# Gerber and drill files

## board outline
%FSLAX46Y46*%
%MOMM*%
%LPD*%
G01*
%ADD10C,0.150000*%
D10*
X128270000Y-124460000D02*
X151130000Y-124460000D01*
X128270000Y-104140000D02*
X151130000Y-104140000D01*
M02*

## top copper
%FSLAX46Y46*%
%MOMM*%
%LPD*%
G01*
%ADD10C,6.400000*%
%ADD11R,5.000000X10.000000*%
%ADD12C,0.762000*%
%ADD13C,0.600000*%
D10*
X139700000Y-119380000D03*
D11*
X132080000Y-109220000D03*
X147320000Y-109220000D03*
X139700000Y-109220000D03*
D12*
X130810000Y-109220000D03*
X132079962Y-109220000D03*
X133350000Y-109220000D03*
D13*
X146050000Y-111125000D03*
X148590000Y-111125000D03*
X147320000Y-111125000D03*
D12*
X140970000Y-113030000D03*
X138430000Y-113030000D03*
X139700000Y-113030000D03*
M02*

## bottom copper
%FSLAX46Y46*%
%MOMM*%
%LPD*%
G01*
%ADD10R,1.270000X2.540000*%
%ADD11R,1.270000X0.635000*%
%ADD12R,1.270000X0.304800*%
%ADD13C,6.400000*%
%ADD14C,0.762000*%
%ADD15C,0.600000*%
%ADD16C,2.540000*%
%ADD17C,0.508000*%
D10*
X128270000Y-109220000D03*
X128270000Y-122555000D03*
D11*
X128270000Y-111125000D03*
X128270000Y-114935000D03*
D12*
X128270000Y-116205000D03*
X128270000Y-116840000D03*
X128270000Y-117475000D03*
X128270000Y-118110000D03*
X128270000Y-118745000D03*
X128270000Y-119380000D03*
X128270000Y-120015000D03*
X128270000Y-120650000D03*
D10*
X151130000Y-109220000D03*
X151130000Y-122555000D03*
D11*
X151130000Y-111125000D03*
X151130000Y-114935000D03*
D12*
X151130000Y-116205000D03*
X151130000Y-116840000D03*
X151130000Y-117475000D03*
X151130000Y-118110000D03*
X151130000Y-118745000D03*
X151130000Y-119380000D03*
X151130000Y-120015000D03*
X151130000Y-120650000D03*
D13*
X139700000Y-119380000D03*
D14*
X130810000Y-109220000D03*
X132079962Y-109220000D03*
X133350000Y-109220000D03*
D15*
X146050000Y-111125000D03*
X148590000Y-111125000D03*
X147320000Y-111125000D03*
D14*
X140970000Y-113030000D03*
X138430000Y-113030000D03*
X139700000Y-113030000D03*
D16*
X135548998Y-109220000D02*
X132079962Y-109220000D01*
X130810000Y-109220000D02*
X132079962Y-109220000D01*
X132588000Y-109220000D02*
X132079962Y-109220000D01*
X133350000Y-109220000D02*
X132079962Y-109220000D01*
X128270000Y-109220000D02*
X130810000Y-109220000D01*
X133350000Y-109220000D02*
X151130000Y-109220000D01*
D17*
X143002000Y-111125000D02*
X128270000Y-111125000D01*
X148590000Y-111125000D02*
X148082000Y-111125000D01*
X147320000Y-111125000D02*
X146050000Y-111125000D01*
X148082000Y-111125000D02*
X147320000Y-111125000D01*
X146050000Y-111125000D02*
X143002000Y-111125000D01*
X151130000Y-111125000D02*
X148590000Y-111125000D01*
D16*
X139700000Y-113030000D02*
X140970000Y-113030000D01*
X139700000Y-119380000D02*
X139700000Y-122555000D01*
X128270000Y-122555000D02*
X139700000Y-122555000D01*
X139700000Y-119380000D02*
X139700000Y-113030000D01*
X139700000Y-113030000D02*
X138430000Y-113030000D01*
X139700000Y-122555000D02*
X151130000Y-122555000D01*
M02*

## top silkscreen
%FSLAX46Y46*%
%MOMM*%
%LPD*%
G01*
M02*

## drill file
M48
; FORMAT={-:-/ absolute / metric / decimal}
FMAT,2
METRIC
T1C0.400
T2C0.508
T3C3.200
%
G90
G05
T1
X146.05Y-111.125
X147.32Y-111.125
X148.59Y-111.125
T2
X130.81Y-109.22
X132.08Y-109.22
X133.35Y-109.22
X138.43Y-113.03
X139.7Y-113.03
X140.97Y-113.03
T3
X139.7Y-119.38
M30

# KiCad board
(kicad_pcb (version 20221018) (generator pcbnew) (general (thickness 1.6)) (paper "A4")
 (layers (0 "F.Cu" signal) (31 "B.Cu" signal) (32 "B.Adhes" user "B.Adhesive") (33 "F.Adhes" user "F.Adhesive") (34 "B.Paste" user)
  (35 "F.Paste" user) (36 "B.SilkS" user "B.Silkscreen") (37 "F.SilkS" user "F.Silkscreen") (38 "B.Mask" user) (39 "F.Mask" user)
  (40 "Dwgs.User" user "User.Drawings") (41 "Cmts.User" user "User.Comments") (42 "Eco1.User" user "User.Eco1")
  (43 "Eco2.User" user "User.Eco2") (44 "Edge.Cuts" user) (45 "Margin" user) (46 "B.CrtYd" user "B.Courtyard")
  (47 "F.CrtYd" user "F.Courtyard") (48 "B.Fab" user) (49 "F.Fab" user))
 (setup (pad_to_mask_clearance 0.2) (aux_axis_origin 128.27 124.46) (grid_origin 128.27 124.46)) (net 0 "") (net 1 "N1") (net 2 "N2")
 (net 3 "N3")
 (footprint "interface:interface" (layer "F.Cu") (at 128.27 104.775)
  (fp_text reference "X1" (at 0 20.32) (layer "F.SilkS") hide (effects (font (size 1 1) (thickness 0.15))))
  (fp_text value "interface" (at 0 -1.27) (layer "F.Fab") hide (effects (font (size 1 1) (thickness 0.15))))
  (pad "1" smd rect (at 0 4.445) (size 1.27 2.54) (layers "B.Cu") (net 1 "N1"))
  (pad "2" smd rect (at 0 17.78) (size 1.27 2.54) (layers "B.Cu") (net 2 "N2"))
  (pad "3" smd rect (at 0 6.35) (size 1.27 0.635) (layers "B.Cu") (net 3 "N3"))
  (pad "4" smd rect (at 0 10.16) (size 1.27 0.635) (layers "B.Cu"))
  (pad "5" smd rect (at 0 11.43) (size 1.27 0.3048) (layers "B.Cu"))
  (pad "6" smd rect (at 0 12.065) (size 1.27 0.3048) (layers "B.Cu"))
  (pad "7" smd rect (at 0 12.7) (size 1.27 0.3048) (layers "B.Cu"))
  (pad "8" smd rect (at 0 13.335) (size 1.27 0.3048) (layers "B.Cu"))
  (pad "9" smd rect (at 0 13.97) (size 1.27 0.3048) (layers "B.Cu"))
  (pad "10" smd rect (at 0 14.605) (size 1.27 0.3048) (layers "B.Cu"))
  (pad "11" smd rect (at 0 15.24) (size 1.27 0.3048) (layers "B.Cu"))
  (pad "12" smd rect (at 0 15.875) (size 1.27 0.3048) (layers "B.Cu")))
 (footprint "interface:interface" (layer "F.Cu") (at 151.13 104.775)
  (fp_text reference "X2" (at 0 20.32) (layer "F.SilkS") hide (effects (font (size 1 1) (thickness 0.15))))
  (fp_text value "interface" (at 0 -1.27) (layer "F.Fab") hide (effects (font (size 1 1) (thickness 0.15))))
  (pad "1" smd rect (at 0 4.445) (size 1.27 2.54) (layers "B.Cu") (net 1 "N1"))
  (pad "2" smd rect (at 0 17.78) (size 1.27 2.54) (layers "B.Cu") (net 2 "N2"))
  (pad "3" smd rect (at 0 6.35) (size 1.27 0.635) (layers "B.Cu") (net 3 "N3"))
  (pad "4" smd rect (at 0 10.16) (size 1.27 0.635) (layers "B.Cu"))
  (pad "5" smd rect (at 0 11.43) (size 1.27 0.3048) (layers "B.Cu"))
  (pad "6" smd rect (at 0 12.065) (size 1.27 0.3048) (layers "B.Cu"))
  (pad "7" smd rect (at 0 12.7) (size 1.27 0.3048) (layers "B.Cu"))
  (pad "8" smd rect (at 0 13.335) (size 1.27 0.3048) (layers "B.Cu"))
  (pad "9" smd rect (at 0 13.97) (size 1.27 0.3048) (layers "B.Cu"))
  (pad "10" smd rect (at 0 14.605) (size 1.27 0.3048) (layers "B.Cu"))
  (pad "11" smd rect (at 0 15.24) (size 1.27 0.3048) (layers "B.Cu"))
  (pad "12" smd rect (at 0 15.875) (size 1.27 0.3048) (layers "B.Cu")))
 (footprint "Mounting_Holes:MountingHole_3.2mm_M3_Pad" (layer "F.Cu") (at 139.7 119.38)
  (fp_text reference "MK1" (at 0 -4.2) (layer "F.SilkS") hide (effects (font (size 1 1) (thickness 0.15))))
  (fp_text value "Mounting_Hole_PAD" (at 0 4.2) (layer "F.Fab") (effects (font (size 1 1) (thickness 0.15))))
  (pad "1" thru_hole circle (at 0 0) (size 6.4 6.4) (drill 3.2) (layers "*.Cu" "*.Mask") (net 2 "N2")))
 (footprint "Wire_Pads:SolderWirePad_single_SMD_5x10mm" (layer "F.Cu") (at 132.08 109.22 180)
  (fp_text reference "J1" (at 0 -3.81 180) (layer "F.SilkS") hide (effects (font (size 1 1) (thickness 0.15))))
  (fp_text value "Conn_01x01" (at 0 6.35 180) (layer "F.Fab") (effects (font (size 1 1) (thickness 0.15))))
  (pad "1" smd rect (at 0 0 180) (size 5 10) (layers "F.Cu" "F.Paste" "F.Mask") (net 1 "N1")))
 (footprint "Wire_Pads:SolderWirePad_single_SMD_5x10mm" (layer "F.Cu") (at 147.32 109.22 180)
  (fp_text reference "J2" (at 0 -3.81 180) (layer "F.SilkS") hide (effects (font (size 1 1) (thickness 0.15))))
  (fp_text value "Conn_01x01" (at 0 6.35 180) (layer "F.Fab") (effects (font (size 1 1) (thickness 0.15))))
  (pad "1" smd rect (at 0 0 180) (size 5 10) (layers "F.Cu" "F.Paste" "F.Mask") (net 3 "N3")))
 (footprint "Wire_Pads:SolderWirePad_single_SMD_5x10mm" (layer "F.Cu") (at 139.7 109.22)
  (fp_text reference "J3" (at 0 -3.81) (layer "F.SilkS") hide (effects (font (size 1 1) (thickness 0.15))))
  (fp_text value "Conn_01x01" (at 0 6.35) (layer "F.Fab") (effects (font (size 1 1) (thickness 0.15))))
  (pad "1" smd rect (at 0 0) (size 5 10) (layers "F.Cu" "F.Paste" "F.Mask") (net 2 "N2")))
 (gr_line (start 128.27 124.46) (end 151.13 124.46) (stroke (width 0.15) (type solid)) (layer "Edge.Cuts"))
 (gr_line (start 128.27 104.14) (end 151.13 104.14) (stroke (width 0.15) (type solid)) (layer "Edge.Cuts"))
 (via (at 130.81 109.22) (size 0.762) (drill 0.508) (layers "F.Cu" "B.Cu") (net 1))
 (via (at 132.079962 109.22) (size 0.762) (drill 0.508) (layers "F.Cu" "B.Cu") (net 1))
 (via (at 133.35 109.22) (size 0.762) (drill 0.508) (layers "F.Cu" "B.Cu") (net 1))
 (segment (start 135.548998 109.22) (end 132.079962 109.22) (width 2.54) (layer "B.Cu") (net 1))
 (segment (start 130.81 109.22) (end 132.079962 109.22) (width 2.54) (layer "B.Cu") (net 1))
 (segment (start 132.588 109.22) (end 132.079962 109.22) (width 2.54) (layer "B.Cu") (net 1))
 (segment (start 133.35 109.22) (end 132.079962 109.22) (width 2.54) (layer "B.Cu") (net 1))
 (segment (start 128.27 109.22) (end 130.81 109.22) (width 2.54) (layer "B.Cu") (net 1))
 (segment (start 133.35 109.22) (end 151.13 109.22) (width 2.54) (layer "B.Cu") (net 1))
 (via (at 146.05 111.125) (size 0.6) (drill 0.4) (layers "F.Cu" "B.Cu") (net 3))
 (via (at 148.59 111.125) (size 0.6) (drill 0.4) (layers "F.Cu" "B.Cu") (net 3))
 (via (at 147.32 111.125) (size 0.6) (drill 0.4) (layers "F.Cu" "B.Cu") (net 3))
 (segment (start 143.002 111.125) (end 128.27 111.125) (width 0.508) (layer "B.Cu") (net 3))
 (segment (start 148.59 111.125) (end 148.082 111.125) (width 0.508) (layer "B.Cu") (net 3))
 (segment (start 147.32 111.125) (end 146.05 111.125) (width 0.508) (layer "B.Cu") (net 3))
 (segment (start 148.082 111.125) (end 147.32 111.125) (width 0.508) (layer "B.Cu") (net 3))
 (segment (start 146.05 111.125) (end 143.002 111.125) (width 0.508) (layer "B.Cu") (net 3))
 (segment (start 151.13 111.125) (end 148.59 111.125) (width 0.508) (layer "B.Cu") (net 3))
 (via (at 140.97 113.03) (size 0.762) (drill 0.508) (layers "F.Cu" "B.Cu") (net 2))
 (via (at 138.43 113.03) (size 0.762) (drill 0.508) (layers "F.Cu" "B.Cu") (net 2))
 (via (at 139.7 113.03) (size 0.762) (drill 0.508) (layers "F.Cu" "B.Cu") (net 2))
 (segment (start 139.7 113.03) (end 140.97 113.03) (width 2.54) (layer "B.Cu") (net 2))
 (segment (start 139.7 119.38) (end 139.7 122.555) (width 2.54) (layer "B.Cu") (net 2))
 (segment (start 128.27 122.555) (end 139.7 122.555) (width 2.54) (layer "B.Cu") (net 2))
 (segment (start 139.7 119.38) (end 139.7 113.03) (width 2.54) (layer "B.Cu") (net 2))
 (segment (start 139.7 113.03) (end 138.43 113.03) (width 2.54) (layer "B.Cu") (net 2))
 (segment (start 139.7 122.555) (end 151.13 122.555) (width 2.54) (layer "B.Cu") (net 2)))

